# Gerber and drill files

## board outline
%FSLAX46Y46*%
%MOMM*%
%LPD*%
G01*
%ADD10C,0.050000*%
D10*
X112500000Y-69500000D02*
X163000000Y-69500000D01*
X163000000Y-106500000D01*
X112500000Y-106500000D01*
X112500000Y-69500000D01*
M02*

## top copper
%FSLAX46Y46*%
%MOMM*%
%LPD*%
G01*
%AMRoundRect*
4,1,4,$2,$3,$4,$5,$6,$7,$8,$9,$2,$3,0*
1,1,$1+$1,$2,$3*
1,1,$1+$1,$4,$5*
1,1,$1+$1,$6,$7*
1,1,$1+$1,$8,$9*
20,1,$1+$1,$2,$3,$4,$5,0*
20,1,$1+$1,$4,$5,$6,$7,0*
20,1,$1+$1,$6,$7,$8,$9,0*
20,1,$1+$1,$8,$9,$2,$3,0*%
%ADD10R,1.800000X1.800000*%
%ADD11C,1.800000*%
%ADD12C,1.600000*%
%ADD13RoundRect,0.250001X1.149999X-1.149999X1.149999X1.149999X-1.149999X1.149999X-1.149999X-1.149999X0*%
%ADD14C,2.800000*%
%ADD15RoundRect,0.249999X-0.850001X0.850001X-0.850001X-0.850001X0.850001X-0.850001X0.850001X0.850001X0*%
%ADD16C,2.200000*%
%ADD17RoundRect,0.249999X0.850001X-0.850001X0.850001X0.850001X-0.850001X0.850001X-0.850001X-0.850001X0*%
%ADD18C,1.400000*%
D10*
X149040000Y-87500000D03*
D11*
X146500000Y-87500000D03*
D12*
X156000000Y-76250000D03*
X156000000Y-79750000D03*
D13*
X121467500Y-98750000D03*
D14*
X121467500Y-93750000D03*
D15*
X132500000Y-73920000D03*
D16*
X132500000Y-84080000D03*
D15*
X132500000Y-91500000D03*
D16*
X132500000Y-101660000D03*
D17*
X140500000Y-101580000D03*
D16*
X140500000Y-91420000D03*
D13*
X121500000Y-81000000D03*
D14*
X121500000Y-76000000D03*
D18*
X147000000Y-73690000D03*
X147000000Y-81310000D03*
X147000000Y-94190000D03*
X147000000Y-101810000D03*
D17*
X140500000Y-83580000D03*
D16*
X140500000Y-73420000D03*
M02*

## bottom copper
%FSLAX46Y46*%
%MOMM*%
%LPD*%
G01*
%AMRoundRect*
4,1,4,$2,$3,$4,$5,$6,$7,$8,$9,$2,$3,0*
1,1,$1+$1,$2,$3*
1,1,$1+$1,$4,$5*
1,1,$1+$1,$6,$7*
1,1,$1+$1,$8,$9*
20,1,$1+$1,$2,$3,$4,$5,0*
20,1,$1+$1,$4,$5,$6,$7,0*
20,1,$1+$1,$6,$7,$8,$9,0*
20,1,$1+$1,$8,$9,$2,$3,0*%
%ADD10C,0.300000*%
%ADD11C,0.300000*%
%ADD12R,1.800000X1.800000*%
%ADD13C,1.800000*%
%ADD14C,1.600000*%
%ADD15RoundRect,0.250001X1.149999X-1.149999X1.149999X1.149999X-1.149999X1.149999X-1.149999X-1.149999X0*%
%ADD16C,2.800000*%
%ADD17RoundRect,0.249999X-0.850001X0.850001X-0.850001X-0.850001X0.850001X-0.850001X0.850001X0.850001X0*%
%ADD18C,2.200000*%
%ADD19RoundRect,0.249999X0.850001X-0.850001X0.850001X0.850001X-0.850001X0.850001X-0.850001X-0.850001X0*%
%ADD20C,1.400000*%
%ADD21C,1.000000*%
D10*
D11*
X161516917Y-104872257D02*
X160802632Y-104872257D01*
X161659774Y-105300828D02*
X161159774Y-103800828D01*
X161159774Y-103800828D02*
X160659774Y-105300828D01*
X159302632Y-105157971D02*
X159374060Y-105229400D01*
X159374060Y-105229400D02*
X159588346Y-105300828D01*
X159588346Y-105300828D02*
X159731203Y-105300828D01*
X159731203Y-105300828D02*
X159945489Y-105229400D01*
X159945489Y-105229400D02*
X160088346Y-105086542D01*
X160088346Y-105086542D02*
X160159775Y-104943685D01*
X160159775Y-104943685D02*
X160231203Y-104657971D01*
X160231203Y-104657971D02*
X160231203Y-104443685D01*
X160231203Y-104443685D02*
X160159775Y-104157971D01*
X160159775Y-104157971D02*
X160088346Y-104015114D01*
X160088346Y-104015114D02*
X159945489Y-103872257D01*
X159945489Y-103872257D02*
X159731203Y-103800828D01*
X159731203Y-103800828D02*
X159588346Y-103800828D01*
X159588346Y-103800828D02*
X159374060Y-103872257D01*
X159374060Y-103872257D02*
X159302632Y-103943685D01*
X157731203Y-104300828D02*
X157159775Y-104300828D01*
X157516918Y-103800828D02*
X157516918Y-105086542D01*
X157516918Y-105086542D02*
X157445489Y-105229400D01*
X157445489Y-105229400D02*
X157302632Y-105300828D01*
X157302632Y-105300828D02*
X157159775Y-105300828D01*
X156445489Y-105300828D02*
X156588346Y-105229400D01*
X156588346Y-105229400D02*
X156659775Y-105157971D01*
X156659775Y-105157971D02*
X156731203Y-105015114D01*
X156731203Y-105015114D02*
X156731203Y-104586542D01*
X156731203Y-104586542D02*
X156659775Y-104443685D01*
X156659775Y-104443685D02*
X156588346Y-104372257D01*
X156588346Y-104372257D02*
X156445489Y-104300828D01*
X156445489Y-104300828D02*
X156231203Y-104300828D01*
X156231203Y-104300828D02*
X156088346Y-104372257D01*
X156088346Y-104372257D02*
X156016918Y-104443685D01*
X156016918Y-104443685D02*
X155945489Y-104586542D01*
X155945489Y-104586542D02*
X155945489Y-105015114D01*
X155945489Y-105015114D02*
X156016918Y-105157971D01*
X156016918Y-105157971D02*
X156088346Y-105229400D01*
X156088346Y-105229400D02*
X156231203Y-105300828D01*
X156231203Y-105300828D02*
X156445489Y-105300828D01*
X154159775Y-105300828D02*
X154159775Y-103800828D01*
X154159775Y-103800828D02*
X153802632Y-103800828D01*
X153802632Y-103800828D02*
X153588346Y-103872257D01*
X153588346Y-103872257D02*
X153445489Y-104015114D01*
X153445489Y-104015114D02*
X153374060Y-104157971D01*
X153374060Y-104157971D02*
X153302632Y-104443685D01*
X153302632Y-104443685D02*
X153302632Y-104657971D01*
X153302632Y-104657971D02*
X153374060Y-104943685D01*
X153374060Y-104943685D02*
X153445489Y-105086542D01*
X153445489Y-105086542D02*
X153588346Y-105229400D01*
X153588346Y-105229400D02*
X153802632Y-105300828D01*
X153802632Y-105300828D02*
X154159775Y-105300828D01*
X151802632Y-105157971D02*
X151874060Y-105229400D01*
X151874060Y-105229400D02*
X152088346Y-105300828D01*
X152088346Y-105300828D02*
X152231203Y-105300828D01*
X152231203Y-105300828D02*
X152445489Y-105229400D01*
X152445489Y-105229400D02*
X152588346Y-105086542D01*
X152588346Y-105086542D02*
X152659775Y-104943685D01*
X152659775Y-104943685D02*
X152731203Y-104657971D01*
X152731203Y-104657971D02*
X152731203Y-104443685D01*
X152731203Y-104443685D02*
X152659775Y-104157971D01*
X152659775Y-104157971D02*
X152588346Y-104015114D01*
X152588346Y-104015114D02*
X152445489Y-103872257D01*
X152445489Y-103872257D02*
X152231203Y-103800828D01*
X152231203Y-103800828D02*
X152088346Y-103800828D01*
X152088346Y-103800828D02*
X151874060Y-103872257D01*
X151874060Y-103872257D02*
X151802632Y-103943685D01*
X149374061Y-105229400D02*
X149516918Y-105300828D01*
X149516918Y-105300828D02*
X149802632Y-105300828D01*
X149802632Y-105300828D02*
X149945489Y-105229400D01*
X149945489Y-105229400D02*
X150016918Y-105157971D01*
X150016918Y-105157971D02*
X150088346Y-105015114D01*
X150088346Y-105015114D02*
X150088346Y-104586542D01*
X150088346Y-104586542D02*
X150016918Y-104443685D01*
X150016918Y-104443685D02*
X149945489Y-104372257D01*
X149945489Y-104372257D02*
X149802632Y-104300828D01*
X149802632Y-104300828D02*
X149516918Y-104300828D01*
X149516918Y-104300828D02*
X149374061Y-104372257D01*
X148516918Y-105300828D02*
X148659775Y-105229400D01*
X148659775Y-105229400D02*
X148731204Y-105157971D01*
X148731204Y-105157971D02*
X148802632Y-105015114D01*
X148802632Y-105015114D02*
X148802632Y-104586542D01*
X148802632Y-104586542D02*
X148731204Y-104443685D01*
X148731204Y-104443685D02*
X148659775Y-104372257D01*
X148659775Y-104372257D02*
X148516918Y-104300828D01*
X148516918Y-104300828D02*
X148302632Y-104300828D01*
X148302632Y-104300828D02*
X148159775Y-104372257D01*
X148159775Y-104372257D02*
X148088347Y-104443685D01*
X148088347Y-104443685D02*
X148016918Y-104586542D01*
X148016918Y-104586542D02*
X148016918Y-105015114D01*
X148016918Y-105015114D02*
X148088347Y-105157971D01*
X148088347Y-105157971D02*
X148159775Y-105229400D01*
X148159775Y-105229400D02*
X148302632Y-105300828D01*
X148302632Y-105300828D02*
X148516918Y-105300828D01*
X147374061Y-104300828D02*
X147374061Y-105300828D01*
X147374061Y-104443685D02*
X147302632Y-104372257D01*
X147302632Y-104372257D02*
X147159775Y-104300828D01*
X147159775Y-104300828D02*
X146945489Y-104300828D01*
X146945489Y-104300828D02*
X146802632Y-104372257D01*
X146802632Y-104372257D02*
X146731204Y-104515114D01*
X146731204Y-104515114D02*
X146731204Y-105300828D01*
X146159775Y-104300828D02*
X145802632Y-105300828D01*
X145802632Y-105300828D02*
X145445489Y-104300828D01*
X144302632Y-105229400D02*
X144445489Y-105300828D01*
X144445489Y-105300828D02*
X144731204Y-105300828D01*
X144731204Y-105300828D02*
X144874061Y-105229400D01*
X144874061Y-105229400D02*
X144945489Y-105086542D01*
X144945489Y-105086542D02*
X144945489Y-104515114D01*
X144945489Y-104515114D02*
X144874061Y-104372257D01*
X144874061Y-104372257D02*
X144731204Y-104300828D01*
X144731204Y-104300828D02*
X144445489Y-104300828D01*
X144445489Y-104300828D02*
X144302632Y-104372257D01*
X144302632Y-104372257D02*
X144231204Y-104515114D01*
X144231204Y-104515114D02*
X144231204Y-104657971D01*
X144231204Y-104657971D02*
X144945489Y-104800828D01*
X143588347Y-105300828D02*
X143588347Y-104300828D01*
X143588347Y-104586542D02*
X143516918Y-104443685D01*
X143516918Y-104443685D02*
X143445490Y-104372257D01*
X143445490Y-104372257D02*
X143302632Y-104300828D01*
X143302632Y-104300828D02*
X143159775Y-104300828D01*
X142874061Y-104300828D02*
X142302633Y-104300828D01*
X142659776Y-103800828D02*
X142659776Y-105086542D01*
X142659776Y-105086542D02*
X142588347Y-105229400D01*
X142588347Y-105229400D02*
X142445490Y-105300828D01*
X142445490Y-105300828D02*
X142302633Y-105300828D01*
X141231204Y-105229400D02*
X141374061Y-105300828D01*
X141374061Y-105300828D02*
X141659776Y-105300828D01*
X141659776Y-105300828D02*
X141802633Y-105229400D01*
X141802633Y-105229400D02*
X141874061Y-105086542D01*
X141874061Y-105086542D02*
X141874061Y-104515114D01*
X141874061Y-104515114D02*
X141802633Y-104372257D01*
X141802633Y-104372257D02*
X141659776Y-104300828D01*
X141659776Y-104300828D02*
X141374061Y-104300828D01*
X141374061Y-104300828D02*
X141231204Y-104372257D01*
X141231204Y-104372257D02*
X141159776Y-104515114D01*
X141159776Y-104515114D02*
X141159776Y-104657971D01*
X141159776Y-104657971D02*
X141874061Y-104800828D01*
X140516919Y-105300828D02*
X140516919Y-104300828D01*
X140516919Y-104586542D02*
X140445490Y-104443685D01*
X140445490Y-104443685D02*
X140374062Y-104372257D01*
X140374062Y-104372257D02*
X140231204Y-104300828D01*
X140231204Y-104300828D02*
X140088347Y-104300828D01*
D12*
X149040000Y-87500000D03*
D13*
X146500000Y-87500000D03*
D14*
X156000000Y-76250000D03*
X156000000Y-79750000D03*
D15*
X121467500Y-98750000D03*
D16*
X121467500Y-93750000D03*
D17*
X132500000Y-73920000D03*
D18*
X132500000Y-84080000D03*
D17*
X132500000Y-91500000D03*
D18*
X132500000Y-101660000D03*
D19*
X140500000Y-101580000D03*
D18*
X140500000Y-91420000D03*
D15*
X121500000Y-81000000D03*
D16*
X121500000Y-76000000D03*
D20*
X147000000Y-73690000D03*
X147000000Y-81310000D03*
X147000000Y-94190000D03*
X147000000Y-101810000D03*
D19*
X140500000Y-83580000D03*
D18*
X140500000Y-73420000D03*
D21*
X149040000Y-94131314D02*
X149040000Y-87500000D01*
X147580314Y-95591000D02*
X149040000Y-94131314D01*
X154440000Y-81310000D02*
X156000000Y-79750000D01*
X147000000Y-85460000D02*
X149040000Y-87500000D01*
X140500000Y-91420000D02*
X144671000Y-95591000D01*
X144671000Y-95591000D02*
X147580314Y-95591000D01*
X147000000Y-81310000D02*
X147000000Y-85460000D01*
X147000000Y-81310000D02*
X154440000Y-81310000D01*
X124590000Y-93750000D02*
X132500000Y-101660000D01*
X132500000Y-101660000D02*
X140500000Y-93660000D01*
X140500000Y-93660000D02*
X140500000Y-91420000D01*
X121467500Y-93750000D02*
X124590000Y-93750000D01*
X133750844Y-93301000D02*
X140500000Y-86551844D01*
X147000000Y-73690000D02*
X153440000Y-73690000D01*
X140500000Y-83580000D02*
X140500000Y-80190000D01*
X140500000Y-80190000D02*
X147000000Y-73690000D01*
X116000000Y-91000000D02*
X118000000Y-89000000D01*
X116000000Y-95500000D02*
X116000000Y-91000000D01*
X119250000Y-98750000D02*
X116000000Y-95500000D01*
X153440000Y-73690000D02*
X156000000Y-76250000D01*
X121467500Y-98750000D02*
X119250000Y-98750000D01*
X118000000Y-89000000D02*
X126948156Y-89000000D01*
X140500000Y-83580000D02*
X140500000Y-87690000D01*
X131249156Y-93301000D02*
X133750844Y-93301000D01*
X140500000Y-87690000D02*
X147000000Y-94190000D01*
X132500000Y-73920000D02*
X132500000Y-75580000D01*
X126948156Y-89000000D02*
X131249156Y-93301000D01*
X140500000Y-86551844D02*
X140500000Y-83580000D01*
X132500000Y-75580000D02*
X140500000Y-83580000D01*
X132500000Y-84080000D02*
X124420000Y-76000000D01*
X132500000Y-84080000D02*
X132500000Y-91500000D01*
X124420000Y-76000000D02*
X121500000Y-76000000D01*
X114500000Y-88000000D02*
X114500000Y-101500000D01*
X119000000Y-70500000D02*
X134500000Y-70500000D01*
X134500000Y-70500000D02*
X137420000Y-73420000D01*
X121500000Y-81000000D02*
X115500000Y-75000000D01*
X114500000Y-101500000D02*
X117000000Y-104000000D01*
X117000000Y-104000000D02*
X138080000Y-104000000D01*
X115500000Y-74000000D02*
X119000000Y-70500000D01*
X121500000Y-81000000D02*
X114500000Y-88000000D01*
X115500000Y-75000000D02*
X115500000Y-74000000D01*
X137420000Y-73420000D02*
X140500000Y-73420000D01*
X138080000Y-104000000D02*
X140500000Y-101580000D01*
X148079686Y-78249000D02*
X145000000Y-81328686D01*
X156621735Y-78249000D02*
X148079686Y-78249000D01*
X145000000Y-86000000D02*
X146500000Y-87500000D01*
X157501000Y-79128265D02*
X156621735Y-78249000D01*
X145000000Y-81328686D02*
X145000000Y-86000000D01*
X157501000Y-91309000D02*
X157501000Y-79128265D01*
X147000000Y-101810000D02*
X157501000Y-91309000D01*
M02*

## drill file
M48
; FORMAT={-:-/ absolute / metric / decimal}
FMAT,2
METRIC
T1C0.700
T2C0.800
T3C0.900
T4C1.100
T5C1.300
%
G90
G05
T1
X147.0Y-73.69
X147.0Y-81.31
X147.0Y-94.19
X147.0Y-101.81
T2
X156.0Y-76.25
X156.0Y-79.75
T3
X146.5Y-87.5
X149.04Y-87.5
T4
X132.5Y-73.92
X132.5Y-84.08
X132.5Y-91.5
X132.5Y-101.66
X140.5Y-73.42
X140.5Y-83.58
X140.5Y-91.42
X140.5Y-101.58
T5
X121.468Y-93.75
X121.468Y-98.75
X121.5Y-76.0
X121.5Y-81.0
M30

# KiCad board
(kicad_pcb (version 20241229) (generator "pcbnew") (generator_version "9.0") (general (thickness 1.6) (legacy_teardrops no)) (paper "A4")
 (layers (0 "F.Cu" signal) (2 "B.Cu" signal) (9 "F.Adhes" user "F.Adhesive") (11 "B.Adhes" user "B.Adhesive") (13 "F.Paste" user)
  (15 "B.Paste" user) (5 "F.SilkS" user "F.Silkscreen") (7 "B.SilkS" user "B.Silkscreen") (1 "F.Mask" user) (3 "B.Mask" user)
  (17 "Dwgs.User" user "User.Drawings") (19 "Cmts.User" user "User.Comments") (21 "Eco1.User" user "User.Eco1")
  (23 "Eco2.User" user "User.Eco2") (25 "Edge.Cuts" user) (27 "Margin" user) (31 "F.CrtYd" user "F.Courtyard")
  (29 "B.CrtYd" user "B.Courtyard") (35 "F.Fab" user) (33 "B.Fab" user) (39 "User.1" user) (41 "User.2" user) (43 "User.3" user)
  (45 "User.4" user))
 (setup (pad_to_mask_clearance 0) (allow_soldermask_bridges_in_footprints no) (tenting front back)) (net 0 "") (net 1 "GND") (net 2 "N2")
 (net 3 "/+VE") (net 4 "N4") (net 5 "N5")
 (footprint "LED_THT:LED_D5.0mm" (layer "F.Cu") (at 149.04 87.5 180)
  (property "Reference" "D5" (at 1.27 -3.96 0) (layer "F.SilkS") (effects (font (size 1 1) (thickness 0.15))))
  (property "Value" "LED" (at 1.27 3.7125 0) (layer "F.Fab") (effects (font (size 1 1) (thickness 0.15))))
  (pad "1" thru_hole rect (at 0 0 180) (size 1.8 1.8) (drill 0.9) (layers "*.Cu" "*.Mask") (remove_unused_layers no) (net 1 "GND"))
  (pad "2" thru_hole circle (at 2.54 0 180) (size 1.8 1.8) (drill 0.9) (layers "*.Cu" "*.Mask") (remove_unused_layers no) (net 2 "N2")))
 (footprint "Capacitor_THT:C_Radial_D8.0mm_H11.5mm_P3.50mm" (layer "F.Cu") (at 156 76.25 -90)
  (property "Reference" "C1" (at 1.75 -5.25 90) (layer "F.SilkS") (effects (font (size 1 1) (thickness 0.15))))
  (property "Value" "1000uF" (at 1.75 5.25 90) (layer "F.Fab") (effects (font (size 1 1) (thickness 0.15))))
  (pad "1" thru_hole circle (at 0 0 270) (size 1.6 1.6) (drill 0.8) (layers "*.Cu" "*.Mask") (remove_unused_layers no) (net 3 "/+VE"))
  (pad "2" thru_hole circle (at 3.5 0 270) (size 1.6 1.6) (drill 0.8) (layers "*.Cu" "*.Mask") (remove_unused_layers no) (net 1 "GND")))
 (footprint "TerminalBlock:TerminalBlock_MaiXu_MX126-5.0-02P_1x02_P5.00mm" (layer "F.Cu") (at 121.4675 98.75 90)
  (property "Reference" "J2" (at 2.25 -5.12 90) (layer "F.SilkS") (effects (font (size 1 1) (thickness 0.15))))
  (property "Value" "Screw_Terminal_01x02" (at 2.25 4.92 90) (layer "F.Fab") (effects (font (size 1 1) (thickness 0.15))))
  (pad "1" thru_hole roundrect (at 0 0 90) (size 2.8 2.8) (drill 1.3) (layers "*.Cu" "*.Mask") (remove_unused_layers no)
   (roundrect_rratio 0.089286) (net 3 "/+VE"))
  (pad "2" thru_hole circle (at 5 0 90) (size 2.8 2.8) (drill 1.3) (layers "*.Cu" "*.Mask") (remove_unused_layers no) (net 1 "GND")))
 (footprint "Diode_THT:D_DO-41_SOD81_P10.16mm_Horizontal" (layer "F.Cu") (at 132.5 73.92 -90)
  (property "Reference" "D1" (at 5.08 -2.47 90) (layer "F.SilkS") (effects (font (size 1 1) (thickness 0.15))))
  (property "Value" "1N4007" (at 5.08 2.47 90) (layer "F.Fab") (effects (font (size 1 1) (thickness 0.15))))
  (pad "1" thru_hole roundrect (at 0 0 270) (size 2.2 2.2) (drill 1.1) (layers "*.Cu" "*.Mask") (remove_unused_layers no)
   (roundrect_rratio 0.113636) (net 3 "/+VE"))
  (pad "2" thru_hole circle (at 10.16 0 270) (size 2.2 2.2) (drill 1.1) (layers "*.Cu" "*.Mask") (remove_unused_layers no) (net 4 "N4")))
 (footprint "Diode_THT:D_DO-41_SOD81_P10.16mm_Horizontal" (layer "F.Cu") (at 132.5 91.5 -90)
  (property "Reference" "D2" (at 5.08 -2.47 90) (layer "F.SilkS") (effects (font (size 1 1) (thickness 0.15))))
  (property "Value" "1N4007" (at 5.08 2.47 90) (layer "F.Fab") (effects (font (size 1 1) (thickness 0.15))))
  (pad "1" thru_hole roundrect (at 0 0 270) (size 2.2 2.2) (drill 1.1) (layers "*.Cu" "*.Mask") (remove_unused_layers no)
   (roundrect_rratio 0.113636) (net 4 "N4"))
  (pad "2" thru_hole circle (at 10.16 0 270) (size 2.2 2.2) (drill 1.1) (layers "*.Cu" "*.Mask") (remove_unused_layers no) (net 1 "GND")))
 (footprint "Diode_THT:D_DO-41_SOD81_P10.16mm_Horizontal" (layer "F.Cu") (at 140.5 101.58 90)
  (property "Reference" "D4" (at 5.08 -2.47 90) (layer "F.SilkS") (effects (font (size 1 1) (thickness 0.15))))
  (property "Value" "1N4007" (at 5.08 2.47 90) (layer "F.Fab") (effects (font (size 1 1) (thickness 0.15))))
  (pad "1" thru_hole roundrect (at 0 0 90) (size 2.2 2.2) (drill 1.1) (layers "*.Cu" "*.Mask") (remove_unused_layers no)
   (roundrect_rratio 0.113636) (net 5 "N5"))
  (pad "2" thru_hole circle (at 10.16 0 90) (size 2.2 2.2) (drill 1.1) (layers "*.Cu" "*.Mask") (remove_unused_layers no) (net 1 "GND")))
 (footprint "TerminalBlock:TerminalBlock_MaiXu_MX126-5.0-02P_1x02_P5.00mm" (layer "F.Cu") (at 121.5 81 90)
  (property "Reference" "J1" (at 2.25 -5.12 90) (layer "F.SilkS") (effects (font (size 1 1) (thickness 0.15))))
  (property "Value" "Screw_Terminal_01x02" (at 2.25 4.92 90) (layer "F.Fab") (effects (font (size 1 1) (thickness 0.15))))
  (pad "1" thru_hole roundrect (at 0 0 90) (size 2.8 2.8) (drill 1.3) (layers "*.Cu" "*.Mask") (remove_unused_layers no)
   (roundrect_rratio 0.089286) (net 5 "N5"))
  (pad "2" thru_hole circle (at 5 0 90) (size 2.8 2.8) (drill 1.3) (layers "*.Cu" "*.Mask") (remove_unused_layers no) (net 4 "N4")))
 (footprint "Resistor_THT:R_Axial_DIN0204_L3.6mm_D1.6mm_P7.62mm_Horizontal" (layer "F.Cu") (at 147 73.69 -90)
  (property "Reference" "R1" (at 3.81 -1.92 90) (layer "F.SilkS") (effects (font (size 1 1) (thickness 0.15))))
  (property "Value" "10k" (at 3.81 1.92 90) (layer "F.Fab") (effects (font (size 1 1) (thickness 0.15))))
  (pad "1" thru_hole circle (at 0 0 270) (size 1.4 1.4) (drill 0.7) (layers "*.Cu" "*.Mask") (remove_unused_layers no) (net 3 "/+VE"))
  (pad "2" thru_hole circle (at 7.62 0 270) (size 1.4 1.4) (drill 0.7) (layers "*.Cu" "*.Mask") (remove_unused_layers no) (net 1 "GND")))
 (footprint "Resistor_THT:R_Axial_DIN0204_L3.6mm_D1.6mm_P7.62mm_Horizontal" (layer "F.Cu") (at 147 94.19 -90)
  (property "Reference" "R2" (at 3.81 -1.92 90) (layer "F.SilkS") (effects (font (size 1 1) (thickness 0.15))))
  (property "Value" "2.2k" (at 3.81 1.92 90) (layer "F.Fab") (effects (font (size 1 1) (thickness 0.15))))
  (pad "1" thru_hole circle (at 0 0 270) (size 1.4 1.4) (drill 0.7) (layers "*.Cu" "*.Mask") (remove_unused_layers no) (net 3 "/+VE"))
  (pad "2" thru_hole circle (at 7.62 0 270) (size 1.4 1.4) (drill 0.7) (layers "*.Cu" "*.Mask") (remove_unused_layers no) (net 2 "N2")))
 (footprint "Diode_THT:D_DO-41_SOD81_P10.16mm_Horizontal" (layer "F.Cu") (at 140.5 83.58 90)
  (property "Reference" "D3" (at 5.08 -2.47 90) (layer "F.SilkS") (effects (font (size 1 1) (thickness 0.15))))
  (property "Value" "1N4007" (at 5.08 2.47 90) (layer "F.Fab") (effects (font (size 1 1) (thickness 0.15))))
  (pad "1" thru_hole roundrect (at 0 0 90) (size 2.2 2.2) (drill 1.1) (layers "*.Cu" "*.Mask") (remove_unused_layers no)
   (roundrect_rratio 0.113636) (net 3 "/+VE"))
  (pad "2" thru_hole circle (at 10.16 0 90) (size 2.2 2.2) (drill 1.1) (layers "*.Cu" "*.Mask") (remove_unused_layers no) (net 5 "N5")))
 (gr_rect (start 112.5 69.5) (end 163 106.5) (stroke (width 0.05) (type default)) (fill no) (layer "Edge.Cuts"))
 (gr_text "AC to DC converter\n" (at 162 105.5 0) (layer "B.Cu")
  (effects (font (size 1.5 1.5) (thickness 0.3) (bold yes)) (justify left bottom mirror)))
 (segment (start 149.04 94.131314) (end 149.04 87.5) (width 1) (layer "B.Cu") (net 1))
 (segment (start 147.580314 95.591) (end 149.04 94.131314) (width 1) (layer "B.Cu") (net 1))
 (segment (start 154.44 81.31) (end 156 79.75) (width 1) (layer "B.Cu") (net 1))
 (segment (start 147 85.46) (end 149.04 87.5) (width 1) (layer "B.Cu") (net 1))
 (segment (start 140.5 91.42) (end 144.671 95.591) (width 1) (layer "B.Cu") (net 1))
 (segment (start 144.671 95.591) (end 147.580314 95.591) (width 1) (layer "B.Cu") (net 1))
 (segment (start 147 81.31) (end 147 85.46) (width 1) (layer "B.Cu") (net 1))
 (segment (start 147 81.31) (end 154.44 81.31) (width 1) (layer "B.Cu") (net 1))
 (segment (start 124.59 93.75) (end 132.5 101.66) (width 1) (layer "B.Cu") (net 1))
 (segment (start 132.5 101.66) (end 140.5 93.66) (width 1) (layer "B.Cu") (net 1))
 (segment (start 140.5 93.66) (end 140.5 91.42) (width 1) (layer "B.Cu") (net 1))
 (segment (start 121.4675 93.75) (end 124.59 93.75) (width 1) (layer "B.Cu") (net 1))
 (segment (start 133.750844 93.301) (end 140.5 86.551844) (width 1) (layer "B.Cu") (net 3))
 (segment (start 147 73.69) (end 153.44 73.69) (width 1) (layer "B.Cu") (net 3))
 (segment (start 140.5 83.58) (end 140.5 80.19) (width 1) (layer "B.Cu") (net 3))
 (segment (start 140.5 80.19) (end 147 73.69) (width 1) (layer "B.Cu") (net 3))
 (segment (start 116 91) (end 118 89) (width 1) (layer "B.Cu") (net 3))
 (segment (start 116 95.5) (end 116 91) (width 1) (layer "B.Cu") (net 3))
 (segment (start 119.25 98.75) (end 116 95.5) (width 1) (layer "B.Cu") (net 3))
 (segment (start 153.44 73.69) (end 156 76.25) (width 1) (layer "B.Cu") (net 3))
 (segment (start 121.4675 98.75) (end 119.25 98.75) (width 1) (layer "B.Cu") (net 3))
 (segment (start 118 89) (end 126.948156 89) (width 1) (layer "B.Cu") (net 3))
 (segment (start 140.5 83.58) (end 140.5 87.69) (width 1) (layer "B.Cu") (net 3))
 (segment (start 131.249156 93.301) (end 133.750844 93.301) (width 1) (layer "B.Cu") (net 3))
 (segment (start 140.5 87.69) (end 147 94.19) (width 1) (layer "B.Cu") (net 3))
 (segment (start 132.5 73.92) (end 132.5 75.58) (width 1) (layer "B.Cu") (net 3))
 (segment (start 126.948156 89) (end 131.249156 93.301) (width 1) (layer "B.Cu") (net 3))
 (segment (start 140.5 86.551844) (end 140.5 83.58) (width 1) (layer "B.Cu") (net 3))
 (segment (start 132.5 75.58) (end 140.5 83.58) (width 1) (layer "B.Cu") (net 3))
 (segment (start 132.5 84.08) (end 124.42 76) (width 1) (layer "B.Cu") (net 4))
 (segment (start 132.5 84.08) (end 132.5 91.5) (width 1) (layer "B.Cu") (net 4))
 (segment (start 124.42 76) (end 121.5 76) (width 1) (layer "B.Cu") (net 4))
 (segment (start 114.5 88) (end 114.5 101.5) (width 1) (layer "B.Cu") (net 5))
 (segment (start 119 70.5) (end 134.5 70.5) (width 1) (layer "B.Cu") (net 5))
 (segment (start 134.5 70.5) (end 137.42 73.42) (width 1) (layer "B.Cu") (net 5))
 (segment (start 121.5 81) (end 115.5 75) (width 1) (layer "B.Cu") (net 5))
 (segment (start 114.5 101.5) (end 117 104) (width 1) (layer "B.Cu") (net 5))
 (segment (start 117 104) (end 138.08 104) (width 1) (layer "B.Cu") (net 5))
 (segment (start 115.5 74) (end 119 70.5) (width 1) (layer "B.Cu") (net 5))
 (segment (start 121.5 81) (end 114.5 88) (width 1) (layer "B.Cu") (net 5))
 (segment (start 115.5 75) (end 115.5 74) (width 1) (layer "B.Cu") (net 5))
 (segment (start 137.42 73.42) (end 140.5 73.42) (width 1) (layer "B.Cu") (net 5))
 (segment (start 138.08 104) (end 140.5 101.58) (width 1) (layer "B.Cu") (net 5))
 (segment (start 148.079686 78.249) (end 145 81.328686) (width 1) (layer "B.Cu") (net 2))
 (segment (start 156.621735 78.249) (end 148.079686 78.249) (width 1) (layer "B.Cu") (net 2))
 (segment (start 145 86) (end 146.5 87.5) (width 1) (layer "B.Cu") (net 2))
 (segment (start 157.501 79.128265) (end 156.621735 78.249) (width 1) (layer "B.Cu") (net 2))
 (segment (start 145 81.328686) (end 145 86) (width 1) (layer "B.Cu") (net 2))
 (segment (start 157.501 91.309) (end 157.501 79.128265) (width 1) (layer "B.Cu") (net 2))
 (segment (start 147 101.81) (end 157.501 91.309) (width 1) (layer "B.Cu") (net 2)))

